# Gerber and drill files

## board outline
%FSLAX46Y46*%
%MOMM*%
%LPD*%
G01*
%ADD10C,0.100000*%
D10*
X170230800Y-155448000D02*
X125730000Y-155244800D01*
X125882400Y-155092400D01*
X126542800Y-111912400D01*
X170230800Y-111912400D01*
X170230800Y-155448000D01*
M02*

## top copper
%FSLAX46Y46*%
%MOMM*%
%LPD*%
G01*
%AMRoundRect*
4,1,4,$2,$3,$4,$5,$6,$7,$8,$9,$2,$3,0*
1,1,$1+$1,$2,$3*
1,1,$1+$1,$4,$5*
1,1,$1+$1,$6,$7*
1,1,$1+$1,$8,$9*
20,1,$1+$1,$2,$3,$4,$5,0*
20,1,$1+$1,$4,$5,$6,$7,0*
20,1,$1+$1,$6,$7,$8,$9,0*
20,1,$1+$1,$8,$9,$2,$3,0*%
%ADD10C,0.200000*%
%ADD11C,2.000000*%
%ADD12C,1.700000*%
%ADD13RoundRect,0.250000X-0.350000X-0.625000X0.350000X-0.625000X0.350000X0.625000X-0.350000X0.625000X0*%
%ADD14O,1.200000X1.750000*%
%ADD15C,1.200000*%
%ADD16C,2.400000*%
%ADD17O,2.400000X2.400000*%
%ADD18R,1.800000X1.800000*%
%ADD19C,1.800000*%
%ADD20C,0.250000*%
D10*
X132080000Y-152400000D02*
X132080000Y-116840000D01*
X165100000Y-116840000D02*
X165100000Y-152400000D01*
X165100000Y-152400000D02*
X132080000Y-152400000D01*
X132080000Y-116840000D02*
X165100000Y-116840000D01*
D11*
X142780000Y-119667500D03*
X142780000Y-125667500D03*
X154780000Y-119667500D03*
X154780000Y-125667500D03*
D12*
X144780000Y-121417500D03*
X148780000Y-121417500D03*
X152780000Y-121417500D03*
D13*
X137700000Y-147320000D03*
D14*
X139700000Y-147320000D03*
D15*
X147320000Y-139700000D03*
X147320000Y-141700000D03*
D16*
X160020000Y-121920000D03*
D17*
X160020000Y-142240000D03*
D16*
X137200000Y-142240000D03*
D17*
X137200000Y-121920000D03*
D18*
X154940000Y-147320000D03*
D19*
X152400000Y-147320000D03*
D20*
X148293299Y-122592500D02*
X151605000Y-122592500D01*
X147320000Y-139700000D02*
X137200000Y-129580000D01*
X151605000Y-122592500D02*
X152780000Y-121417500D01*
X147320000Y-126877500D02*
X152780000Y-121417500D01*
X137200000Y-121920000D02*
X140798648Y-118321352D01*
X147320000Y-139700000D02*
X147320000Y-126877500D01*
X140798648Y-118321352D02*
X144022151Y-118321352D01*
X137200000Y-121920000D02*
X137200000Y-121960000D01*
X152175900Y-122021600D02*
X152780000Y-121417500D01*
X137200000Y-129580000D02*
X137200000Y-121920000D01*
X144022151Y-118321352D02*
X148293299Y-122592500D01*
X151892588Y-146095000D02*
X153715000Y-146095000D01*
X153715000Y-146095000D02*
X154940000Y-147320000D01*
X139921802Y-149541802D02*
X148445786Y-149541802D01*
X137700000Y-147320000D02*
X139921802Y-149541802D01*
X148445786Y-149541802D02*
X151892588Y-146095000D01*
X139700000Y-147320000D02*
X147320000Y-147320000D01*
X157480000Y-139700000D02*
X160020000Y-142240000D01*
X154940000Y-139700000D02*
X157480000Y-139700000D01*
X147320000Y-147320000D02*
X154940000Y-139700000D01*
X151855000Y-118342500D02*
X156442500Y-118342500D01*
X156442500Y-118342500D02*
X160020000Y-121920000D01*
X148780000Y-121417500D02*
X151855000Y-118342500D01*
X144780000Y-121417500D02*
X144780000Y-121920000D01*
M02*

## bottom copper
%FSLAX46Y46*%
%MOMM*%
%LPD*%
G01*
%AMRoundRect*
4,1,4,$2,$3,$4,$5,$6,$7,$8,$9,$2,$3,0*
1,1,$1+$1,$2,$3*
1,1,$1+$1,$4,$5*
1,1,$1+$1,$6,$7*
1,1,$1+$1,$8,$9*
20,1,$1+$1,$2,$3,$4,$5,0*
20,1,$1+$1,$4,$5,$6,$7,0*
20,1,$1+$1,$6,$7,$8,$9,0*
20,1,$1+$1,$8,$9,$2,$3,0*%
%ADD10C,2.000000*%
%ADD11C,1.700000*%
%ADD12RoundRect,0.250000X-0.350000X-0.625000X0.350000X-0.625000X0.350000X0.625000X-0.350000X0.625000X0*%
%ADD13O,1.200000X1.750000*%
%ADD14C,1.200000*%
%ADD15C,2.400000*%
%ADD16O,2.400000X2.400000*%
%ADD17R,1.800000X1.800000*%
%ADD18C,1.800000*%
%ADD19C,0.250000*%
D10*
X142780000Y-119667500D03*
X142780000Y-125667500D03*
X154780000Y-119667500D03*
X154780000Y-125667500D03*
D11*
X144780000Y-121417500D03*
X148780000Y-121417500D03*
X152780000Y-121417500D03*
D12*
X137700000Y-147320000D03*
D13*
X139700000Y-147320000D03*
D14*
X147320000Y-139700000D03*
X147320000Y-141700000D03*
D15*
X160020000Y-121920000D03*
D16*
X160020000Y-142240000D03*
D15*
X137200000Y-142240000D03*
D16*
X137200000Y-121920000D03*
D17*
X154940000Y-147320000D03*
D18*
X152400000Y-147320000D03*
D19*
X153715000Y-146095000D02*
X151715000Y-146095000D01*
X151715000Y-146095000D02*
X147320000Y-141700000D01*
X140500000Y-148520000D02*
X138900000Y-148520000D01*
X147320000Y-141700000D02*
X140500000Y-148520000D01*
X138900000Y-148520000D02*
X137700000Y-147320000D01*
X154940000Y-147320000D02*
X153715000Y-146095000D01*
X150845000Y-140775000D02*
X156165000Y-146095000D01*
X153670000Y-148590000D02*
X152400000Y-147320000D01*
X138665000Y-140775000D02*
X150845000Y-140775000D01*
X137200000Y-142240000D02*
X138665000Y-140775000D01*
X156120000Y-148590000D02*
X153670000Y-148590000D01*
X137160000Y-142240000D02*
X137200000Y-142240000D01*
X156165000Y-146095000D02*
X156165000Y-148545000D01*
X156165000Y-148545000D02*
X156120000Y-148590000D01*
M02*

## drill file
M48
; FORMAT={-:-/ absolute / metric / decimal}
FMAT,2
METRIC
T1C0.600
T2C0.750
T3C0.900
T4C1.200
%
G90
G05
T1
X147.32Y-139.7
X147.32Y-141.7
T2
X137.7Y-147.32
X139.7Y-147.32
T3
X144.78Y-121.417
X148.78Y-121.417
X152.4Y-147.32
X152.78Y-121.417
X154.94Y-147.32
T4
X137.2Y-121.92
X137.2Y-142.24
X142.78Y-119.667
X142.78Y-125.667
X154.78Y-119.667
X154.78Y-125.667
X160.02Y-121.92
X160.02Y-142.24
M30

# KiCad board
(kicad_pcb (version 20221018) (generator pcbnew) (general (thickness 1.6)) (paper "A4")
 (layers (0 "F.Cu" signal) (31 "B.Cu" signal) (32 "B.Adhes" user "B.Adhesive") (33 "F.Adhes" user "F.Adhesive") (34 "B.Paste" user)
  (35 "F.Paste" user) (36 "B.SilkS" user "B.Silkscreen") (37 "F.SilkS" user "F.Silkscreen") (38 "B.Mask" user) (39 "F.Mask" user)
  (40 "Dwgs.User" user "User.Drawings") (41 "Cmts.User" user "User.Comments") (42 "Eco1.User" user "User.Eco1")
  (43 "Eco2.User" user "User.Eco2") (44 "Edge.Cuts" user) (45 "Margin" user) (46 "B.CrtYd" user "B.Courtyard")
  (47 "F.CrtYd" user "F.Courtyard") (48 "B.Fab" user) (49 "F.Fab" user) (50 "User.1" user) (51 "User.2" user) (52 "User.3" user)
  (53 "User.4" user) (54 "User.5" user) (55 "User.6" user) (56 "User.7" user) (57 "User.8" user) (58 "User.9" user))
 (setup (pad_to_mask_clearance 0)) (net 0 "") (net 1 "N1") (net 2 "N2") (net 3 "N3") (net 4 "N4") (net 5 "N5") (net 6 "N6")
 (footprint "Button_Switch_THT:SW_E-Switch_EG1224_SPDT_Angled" (layer "F.Cu") (at 144.78 121.4175)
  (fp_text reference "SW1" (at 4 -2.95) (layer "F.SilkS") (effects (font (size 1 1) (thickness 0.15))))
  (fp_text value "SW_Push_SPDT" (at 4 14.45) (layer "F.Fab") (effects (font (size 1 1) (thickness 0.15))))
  (pad "" thru_hole circle (at -2 -1.75) (size 2 2) (drill 1.2) (layers "*.Cu" "*.Mask"))
  (pad "" thru_hole circle (at -2 4.25) (size 2 2) (drill 1.2) (layers "*.Cu" "*.Mask"))
  (pad "" thru_hole circle (at 10 -1.75) (size 2 2) (drill 1.2) (layers "*.Cu" "*.Mask"))
  (pad "" thru_hole circle (at 10 4.25) (size 2 2) (drill 1.2) (layers "*.Cu" "*.Mask"))
  (pad "1" thru_hole circle (at 0 0) (size 1.7 1.7) (drill 0.9) (layers "*.Cu" "*.Mask") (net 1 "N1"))
  (pad "2" thru_hole circle (at 4 0) (size 1.7 1.7) (drill 0.9) (layers "*.Cu" "*.Mask") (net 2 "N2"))
  (pad "3" thru_hole circle (at 8 0) (size 1.7 1.7) (drill 0.9) (layers "*.Cu" "*.Mask") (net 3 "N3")))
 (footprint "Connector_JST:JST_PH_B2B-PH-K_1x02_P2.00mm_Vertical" (layer "F.Cu") (at 137.7 147.32)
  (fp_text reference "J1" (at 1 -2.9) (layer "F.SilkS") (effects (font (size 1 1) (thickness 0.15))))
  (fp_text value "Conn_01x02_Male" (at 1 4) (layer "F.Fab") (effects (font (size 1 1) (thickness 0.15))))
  (pad "1" thru_hole roundrect (at 0 0) (size 1.2 1.75) (drill 0.75) (layers "*.Cu" "*.Mask") (roundrect_rratio 0.208333) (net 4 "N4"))
  (pad "2" thru_hole oval (at 2 0) (size 1.2 1.75) (drill 0.75) (layers "*.Cu" "*.Mask") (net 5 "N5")))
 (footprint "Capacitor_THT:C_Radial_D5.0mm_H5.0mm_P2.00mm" (layer "F.Cu") (at 147.32 139.7 -90)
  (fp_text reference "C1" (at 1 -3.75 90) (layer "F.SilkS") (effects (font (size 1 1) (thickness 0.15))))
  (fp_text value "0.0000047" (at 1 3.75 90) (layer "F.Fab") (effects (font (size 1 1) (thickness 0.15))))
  (pad "1" thru_hole circle (at 0 0 270) (size 1.2 1.2) (drill 0.6) (layers "*.Cu" "*.Mask") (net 3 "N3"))
  (pad "2" thru_hole circle (at 2 0 270) (size 1.2 1.2) (drill 0.6) (layers "*.Cu" "*.Mask") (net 4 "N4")))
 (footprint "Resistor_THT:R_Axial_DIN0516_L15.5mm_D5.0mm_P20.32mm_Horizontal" (layer "F.Cu") (at 160.02 121.92 -90)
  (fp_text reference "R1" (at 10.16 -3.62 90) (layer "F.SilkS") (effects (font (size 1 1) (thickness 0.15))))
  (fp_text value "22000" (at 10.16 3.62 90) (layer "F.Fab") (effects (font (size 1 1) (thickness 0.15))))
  (pad "1" thru_hole circle (at 0 0 270) (size 2.4 2.4) (drill 1.2) (layers "*.Cu" "*.Mask") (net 2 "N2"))
  (pad "2" thru_hole oval (at 20.32 0 270) (size 2.4 2.4) (drill 1.2) (layers "*.Cu" "*.Mask") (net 5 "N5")))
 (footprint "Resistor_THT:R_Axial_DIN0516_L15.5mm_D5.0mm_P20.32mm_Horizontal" (layer "F.Cu") (at 137.2 142.24 90)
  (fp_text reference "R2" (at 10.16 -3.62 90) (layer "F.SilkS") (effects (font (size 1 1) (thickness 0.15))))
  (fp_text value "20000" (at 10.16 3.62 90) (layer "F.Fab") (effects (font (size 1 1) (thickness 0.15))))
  (pad "1" thru_hole circle (at 0 0 90) (size 2.4 2.4) (drill 1.2) (layers "*.Cu" "*.Mask") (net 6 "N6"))
  (pad "2" thru_hole oval (at 20.32 0 90) (size 2.4 2.4) (drill 1.2) (layers "*.Cu" "*.Mask") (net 3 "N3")))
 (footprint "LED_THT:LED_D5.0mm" (layer "F.Cu") (at 154.94 147.32 180)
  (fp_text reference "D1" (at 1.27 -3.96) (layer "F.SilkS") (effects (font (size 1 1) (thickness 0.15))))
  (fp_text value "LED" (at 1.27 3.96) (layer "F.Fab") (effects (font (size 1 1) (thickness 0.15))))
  (pad "1" thru_hole rect (at 0 0 180) (size 1.8 1.8) (drill 0.9) (layers "*.Cu" "*.Mask") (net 4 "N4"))
  (pad "2" thru_hole circle (at 2.54 0 180) (size 1.8 1.8) (drill 0.9) (layers "*.Cu" "*.Mask") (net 6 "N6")))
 (gr_line (start 132.08 152.4) (end 132.08 116.84) (stroke (width 0.2) (type solid)) (layer "F.Cu"))
 (gr_line (start 165.1 116.84) (end 165.1 152.4) (stroke (width 0.2) (type solid)) (layer "F.Cu"))
 (gr_line (start 165.1 152.4) (end 132.08 152.4) (stroke (width 0.2) (type solid)) (layer "F.Cu"))
 (gr_line (start 132.08 116.84) (end 165.1 116.84) (stroke (width 0.2) (type solid)) (layer "F.Cu"))
 (gr_poly
  (pts (xy 170.2308 155.448) (xy 125.73 155.2448) (xy 125.8824 155.0924) (xy 126.5428 111.9124) (xy 170.2308 111.9124))
  (stroke (width 0.1) (type solid)) (fill none) (layer "Edge.Cuts"))
 (segment (start 148.293299 122.5925) (end 151.605 122.5925) (width 0.25) (layer "F.Cu") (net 3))
 (segment (start 147.32 139.7) (end 137.2 129.58) (width 0.25) (layer "F.Cu") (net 3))
 (segment (start 151.605 122.5925) (end 152.78 121.4175) (width 0.25) (layer "F.Cu") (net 3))
 (segment (start 147.32 126.8775) (end 152.78 121.4175) (width 0.25) (layer "F.Cu") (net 3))
 (segment (start 137.2 121.92) (end 140.798648 118.321352) (width 0.25) (layer "F.Cu") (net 3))
 (segment (start 147.32 139.7) (end 147.32 126.8775) (width 0.25) (layer "F.Cu") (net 3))
 (segment (start 140.798648 118.321352) (end 144.022151 118.321352) (width 0.25) (layer "F.Cu") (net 3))
 (segment (start 137.2 121.92) (end 137.2 121.96) (width 0.25) (layer "F.Cu") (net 3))
 (segment (start 152.1759 122.0216) (end 152.78 121.4175) (width 0.25) (layer "F.Cu") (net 3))
 (segment (start 137.2 129.58) (end 137.2 121.92) (width 0.25) (layer "F.Cu") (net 3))
 (segment (start 144.022151 118.321352) (end 148.293299 122.5925) (width 0.25) (layer "F.Cu") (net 3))
 (segment (start 151.892588 146.095) (end 153.715 146.095) (width 0.25) (layer "F.Cu") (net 4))
 (segment (start 153.715 146.095) (end 154.94 147.32) (width 0.25) (layer "F.Cu") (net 4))
 (segment (start 139.921802 149.541802) (end 148.445786 149.541802) (width 0.25) (layer "F.Cu") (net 4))
 (segment (start 137.7 147.32) (end 139.921802 149.541802) (width 0.25) (layer "F.Cu") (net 4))
 (segment (start 148.445786 149.541802) (end 151.892588 146.095) (width 0.25) (layer "F.Cu") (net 4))
 (segment (start 153.715 146.095) (end 151.715 146.095) (width 0.25) (layer "B.Cu") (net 4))
 (segment (start 151.715 146.095) (end 147.32 141.7) (width 0.25) (layer "B.Cu") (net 4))
 (segment (start 140.5 148.52) (end 138.9 148.52) (width 0.25) (layer "B.Cu") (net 4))
 (segment (start 147.32 141.7) (end 140.5 148.52) (width 0.25) (layer "B.Cu") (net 4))
 (segment (start 138.9 148.52) (end 137.7 147.32) (width 0.25) (layer "B.Cu") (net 4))
 (segment (start 154.94 147.32) (end 153.715 146.095) (width 0.25) (layer "B.Cu") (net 4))
 (segment (start 150.845 140.775) (end 156.165 146.095) (width 0.25) (layer "B.Cu") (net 6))
 (segment (start 153.67 148.59) (end 152.4 147.32) (width 0.25) (layer "B.Cu") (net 6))
 (segment (start 138.665 140.775) (end 150.845 140.775) (width 0.25) (layer "B.Cu") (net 6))
 (segment (start 137.2 142.24) (end 138.665 140.775) (width 0.25) (layer "B.Cu") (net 6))
 (segment (start 156.12 148.59) (end 153.67 148.59) (width 0.25) (layer "B.Cu") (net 6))
 (segment (start 137.16 142.24) (end 137.2 142.24) (width 0.25) (layer "B.Cu") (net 6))
 (segment (start 156.165 146.095) (end 156.165 148.545) (width 0.25) (layer "B.Cu") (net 6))
 (segment (start 156.165 148.545) (end 156.12 148.59) (width 0.25) (layer "B.Cu") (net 6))
 (segment (start 139.7 147.32) (end 147.32 147.32) (width 0.25) (layer "F.Cu") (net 5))
 (segment (start 157.48 139.7) (end 160.02 142.24) (width 0.25) (layer "F.Cu") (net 5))
 (segment (start 154.94 139.7) (end 157.48 139.7) (width 0.25) (layer "F.Cu") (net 5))
 (segment (start 147.32 147.32) (end 154.94 139.7) (width 0.25) (layer "F.Cu") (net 5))
 (segment (start 151.855 118.3425) (end 156.4425 118.3425) (width 0.25) (layer "F.Cu") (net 2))
 (segment (start 156.4425 118.3425) (end 160.02 121.92) (width 0.25) (layer "F.Cu") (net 2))
 (segment (start 148.78 121.4175) (end 151.855 118.3425) (width 0.25) (layer "F.Cu") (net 2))
 (segment (start 144.78 121.4175) (end 144.78 121.92) (width 0.25) (layer "F.Cu") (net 1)))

